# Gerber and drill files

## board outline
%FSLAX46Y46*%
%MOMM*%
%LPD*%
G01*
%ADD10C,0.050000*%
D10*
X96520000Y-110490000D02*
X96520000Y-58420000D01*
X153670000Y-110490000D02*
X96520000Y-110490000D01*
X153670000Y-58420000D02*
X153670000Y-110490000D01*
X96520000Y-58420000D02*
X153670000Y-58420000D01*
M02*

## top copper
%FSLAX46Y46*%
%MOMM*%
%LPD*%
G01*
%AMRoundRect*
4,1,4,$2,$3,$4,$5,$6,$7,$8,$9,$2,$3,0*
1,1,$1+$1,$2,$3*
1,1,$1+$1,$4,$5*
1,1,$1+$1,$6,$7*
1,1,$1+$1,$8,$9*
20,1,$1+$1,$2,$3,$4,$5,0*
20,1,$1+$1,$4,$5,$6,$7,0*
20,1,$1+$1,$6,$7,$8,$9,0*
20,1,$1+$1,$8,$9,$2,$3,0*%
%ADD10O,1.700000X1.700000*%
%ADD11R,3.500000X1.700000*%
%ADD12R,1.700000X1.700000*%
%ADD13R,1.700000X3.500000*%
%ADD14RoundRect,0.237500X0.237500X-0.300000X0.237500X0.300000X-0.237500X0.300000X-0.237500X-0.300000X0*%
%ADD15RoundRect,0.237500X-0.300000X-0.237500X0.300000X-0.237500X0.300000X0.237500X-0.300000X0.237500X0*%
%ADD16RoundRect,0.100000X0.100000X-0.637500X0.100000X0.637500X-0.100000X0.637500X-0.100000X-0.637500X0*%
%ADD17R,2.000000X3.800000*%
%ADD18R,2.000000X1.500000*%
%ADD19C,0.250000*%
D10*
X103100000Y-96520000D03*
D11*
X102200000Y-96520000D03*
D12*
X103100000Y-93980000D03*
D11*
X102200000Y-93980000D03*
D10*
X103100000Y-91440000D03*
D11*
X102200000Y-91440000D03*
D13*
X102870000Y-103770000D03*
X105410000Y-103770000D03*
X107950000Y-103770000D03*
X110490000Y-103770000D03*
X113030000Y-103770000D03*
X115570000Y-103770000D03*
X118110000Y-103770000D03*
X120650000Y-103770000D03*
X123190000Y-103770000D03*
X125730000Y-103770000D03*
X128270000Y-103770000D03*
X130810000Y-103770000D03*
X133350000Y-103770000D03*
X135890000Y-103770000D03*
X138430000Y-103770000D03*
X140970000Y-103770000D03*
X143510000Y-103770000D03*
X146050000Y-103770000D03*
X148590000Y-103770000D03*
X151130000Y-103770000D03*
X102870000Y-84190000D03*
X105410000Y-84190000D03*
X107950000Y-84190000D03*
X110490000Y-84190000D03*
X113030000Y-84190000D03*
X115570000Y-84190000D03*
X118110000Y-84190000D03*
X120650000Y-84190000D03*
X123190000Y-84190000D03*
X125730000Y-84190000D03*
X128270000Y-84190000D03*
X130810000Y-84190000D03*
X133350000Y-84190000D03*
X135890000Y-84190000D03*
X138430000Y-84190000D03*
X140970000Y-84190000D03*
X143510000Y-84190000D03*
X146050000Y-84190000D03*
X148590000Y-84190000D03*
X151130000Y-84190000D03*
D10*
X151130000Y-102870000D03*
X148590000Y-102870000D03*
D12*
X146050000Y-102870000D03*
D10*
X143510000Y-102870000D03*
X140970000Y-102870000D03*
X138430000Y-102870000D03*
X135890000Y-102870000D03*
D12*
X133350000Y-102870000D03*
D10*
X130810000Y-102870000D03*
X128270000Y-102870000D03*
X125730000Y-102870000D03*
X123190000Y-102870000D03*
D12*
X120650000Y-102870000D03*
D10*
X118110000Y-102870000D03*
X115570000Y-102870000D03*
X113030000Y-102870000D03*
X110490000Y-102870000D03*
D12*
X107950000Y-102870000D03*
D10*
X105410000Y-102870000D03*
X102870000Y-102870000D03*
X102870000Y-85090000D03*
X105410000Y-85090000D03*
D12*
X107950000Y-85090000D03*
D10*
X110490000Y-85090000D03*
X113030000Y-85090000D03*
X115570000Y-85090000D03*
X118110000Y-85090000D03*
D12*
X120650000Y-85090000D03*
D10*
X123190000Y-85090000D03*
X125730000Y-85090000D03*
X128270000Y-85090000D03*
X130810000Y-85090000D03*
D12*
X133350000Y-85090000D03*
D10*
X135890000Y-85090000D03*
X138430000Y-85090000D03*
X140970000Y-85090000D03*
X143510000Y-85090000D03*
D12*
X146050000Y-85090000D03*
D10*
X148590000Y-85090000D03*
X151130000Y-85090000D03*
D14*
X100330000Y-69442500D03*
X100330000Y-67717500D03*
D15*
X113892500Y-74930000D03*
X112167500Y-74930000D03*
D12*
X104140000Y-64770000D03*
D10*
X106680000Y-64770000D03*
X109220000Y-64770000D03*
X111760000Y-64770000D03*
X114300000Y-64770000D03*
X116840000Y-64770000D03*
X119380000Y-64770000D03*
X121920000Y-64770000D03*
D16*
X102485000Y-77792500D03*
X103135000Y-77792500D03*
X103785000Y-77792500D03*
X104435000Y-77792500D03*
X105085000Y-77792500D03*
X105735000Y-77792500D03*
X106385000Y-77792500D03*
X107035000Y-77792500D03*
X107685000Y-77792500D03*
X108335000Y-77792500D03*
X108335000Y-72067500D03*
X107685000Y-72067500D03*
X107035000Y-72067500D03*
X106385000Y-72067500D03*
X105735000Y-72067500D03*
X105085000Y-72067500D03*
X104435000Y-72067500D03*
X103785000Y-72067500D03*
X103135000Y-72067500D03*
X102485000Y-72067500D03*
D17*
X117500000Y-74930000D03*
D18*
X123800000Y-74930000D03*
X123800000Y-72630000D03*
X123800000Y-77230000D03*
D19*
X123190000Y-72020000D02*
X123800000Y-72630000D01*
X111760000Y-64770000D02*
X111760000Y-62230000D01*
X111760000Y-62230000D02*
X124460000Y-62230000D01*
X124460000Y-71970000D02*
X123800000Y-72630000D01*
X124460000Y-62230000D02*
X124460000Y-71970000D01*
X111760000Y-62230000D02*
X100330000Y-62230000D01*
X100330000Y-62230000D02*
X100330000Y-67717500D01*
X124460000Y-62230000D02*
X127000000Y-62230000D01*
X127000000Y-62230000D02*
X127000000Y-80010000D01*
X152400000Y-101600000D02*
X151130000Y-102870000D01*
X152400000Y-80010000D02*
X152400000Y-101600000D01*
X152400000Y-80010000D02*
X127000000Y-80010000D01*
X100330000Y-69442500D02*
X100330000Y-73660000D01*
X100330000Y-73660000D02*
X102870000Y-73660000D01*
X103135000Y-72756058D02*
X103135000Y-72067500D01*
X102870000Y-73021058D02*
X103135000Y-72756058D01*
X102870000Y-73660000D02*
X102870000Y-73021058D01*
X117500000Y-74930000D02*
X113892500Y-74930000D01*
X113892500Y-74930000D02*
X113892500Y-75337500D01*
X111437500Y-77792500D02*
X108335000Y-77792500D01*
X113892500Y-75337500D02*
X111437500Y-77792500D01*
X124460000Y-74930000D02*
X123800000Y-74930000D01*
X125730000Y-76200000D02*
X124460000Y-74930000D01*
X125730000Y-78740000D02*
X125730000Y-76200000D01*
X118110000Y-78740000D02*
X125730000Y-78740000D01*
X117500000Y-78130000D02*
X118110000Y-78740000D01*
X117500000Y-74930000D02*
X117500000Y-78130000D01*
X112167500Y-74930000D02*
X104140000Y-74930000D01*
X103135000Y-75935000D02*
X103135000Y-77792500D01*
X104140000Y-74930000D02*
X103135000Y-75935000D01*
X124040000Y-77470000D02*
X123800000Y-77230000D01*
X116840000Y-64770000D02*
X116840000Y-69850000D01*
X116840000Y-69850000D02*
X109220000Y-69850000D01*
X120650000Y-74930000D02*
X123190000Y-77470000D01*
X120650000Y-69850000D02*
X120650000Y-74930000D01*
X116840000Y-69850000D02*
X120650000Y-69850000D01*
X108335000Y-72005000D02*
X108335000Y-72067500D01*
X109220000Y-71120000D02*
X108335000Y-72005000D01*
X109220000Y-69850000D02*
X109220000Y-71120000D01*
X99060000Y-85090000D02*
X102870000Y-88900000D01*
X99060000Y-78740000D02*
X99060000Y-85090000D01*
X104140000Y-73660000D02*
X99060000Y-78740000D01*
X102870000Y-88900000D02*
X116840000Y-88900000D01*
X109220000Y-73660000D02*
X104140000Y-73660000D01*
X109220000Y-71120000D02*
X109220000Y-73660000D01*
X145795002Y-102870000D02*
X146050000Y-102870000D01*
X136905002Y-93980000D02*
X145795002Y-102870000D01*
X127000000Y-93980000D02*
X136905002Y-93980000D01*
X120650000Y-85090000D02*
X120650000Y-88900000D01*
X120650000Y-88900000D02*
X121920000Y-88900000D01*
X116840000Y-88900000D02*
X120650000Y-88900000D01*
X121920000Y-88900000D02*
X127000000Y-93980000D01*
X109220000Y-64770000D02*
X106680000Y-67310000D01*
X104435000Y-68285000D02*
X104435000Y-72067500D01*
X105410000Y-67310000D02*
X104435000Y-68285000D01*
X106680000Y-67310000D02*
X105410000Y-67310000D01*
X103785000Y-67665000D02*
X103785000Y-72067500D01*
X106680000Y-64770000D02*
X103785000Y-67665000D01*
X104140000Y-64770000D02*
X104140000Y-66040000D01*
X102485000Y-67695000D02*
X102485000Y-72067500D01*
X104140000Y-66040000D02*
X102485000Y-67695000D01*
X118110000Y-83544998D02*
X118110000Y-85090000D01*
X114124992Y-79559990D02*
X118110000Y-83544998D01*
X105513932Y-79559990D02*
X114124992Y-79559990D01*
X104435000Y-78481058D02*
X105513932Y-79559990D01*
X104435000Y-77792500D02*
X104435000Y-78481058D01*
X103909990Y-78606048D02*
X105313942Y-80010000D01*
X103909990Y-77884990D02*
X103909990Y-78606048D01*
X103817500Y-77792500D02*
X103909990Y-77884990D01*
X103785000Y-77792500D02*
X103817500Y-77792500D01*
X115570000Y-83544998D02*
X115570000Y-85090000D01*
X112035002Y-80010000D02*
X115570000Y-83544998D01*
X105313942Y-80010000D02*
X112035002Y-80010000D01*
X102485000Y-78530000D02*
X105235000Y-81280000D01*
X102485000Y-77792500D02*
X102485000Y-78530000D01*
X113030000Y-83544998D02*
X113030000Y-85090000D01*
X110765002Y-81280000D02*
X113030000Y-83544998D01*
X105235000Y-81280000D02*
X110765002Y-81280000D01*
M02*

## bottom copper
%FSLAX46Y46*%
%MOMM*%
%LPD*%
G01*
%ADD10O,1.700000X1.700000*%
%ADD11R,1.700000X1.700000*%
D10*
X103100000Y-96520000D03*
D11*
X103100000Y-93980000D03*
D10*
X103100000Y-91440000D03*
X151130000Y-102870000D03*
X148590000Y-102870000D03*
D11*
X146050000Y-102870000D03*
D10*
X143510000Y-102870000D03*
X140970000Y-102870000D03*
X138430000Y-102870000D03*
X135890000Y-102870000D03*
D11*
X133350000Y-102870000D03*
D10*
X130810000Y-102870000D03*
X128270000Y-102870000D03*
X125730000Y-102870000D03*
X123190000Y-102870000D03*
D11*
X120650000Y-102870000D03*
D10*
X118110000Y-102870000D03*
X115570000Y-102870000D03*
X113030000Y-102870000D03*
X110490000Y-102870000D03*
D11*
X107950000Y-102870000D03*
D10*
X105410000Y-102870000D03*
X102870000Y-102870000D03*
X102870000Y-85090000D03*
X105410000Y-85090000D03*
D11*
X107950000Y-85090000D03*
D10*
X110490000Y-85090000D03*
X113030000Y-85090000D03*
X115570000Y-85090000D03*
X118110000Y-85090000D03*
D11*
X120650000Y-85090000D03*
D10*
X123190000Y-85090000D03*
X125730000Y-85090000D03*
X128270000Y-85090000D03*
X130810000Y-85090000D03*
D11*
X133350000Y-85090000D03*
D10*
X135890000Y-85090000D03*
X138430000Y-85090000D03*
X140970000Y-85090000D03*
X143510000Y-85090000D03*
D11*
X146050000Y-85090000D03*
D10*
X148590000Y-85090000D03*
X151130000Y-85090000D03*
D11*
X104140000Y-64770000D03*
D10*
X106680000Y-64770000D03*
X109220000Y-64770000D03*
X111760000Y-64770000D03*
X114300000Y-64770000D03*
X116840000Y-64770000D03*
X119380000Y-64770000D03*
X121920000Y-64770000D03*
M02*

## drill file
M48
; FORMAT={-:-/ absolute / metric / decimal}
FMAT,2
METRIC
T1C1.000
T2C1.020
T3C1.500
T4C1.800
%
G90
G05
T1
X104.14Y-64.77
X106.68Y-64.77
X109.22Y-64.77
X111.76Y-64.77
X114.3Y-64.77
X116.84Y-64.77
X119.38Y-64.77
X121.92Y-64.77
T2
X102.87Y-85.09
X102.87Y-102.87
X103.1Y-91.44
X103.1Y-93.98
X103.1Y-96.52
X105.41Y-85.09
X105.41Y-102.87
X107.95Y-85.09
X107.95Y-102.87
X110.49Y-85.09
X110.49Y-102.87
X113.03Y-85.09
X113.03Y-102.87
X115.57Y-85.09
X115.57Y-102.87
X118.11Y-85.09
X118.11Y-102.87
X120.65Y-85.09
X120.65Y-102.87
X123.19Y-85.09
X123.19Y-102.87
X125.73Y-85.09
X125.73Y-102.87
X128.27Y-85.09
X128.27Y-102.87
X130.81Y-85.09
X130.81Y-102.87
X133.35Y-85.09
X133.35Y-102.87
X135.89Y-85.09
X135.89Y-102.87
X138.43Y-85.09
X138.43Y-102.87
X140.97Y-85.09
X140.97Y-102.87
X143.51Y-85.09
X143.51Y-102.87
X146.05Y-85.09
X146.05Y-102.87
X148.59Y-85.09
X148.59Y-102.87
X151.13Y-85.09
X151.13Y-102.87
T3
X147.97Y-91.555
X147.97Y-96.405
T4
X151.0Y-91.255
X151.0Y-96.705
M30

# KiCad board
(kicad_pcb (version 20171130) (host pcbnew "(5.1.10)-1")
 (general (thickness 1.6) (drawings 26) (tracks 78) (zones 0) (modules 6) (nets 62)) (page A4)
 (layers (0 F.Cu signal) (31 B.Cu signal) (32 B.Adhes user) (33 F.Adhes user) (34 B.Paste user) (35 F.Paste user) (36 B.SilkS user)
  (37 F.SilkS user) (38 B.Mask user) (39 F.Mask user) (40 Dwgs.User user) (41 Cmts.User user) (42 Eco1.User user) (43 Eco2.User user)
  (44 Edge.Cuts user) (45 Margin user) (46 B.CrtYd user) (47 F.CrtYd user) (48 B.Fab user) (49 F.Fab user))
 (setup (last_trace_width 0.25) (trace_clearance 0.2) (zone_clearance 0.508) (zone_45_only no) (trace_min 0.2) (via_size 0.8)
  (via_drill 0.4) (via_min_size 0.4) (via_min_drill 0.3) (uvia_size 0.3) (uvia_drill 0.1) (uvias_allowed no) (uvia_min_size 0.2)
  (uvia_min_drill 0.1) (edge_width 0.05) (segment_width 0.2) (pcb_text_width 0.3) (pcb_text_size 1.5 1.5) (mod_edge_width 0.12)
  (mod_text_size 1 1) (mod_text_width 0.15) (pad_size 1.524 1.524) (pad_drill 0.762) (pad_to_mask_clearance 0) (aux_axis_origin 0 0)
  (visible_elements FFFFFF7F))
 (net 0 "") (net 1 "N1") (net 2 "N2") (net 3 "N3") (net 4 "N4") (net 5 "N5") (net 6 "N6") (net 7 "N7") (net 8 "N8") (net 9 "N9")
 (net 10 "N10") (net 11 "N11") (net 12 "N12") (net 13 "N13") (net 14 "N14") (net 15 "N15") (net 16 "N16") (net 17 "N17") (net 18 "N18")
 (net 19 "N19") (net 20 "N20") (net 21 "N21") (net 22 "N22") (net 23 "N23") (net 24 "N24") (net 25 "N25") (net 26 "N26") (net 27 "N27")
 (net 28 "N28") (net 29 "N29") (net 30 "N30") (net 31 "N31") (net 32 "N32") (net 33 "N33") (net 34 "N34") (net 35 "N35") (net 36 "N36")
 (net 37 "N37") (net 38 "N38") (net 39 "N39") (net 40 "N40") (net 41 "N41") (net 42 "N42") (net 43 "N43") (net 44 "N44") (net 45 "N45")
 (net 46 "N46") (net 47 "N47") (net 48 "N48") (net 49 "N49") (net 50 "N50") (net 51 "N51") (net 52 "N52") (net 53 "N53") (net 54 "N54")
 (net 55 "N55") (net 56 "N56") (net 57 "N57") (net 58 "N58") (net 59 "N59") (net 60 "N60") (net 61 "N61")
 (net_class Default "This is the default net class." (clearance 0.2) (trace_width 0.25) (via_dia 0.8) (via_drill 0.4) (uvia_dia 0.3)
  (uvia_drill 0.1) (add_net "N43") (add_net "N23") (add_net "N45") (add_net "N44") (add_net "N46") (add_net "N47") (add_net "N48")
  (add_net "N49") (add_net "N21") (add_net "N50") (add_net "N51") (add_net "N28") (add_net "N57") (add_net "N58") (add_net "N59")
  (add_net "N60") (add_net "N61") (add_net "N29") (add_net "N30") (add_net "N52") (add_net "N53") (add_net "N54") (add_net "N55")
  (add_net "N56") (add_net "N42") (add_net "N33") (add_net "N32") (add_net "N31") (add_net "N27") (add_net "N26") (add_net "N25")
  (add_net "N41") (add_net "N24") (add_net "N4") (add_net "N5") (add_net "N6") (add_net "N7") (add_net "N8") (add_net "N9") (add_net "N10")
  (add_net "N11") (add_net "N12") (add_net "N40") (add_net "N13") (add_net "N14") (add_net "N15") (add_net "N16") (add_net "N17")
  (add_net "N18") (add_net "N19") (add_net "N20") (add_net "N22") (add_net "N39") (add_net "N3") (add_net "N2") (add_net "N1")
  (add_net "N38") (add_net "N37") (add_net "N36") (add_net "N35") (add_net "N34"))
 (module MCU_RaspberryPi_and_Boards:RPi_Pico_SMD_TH (layer F.Cu) (at 127 93.98 270)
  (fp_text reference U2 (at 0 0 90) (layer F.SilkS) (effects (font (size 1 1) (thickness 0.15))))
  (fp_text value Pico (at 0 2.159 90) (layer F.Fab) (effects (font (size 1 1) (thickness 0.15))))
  (pad 43 thru_hole oval (at 2.54 23.9 270) (size 1.7 1.7) (drill 1.02) (layers *.Cu *.Mask) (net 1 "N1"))
  (pad 43 smd rect (at 2.54 23.9) (size 3.5 1.7) (drill (offset -0.9 0)) (layers F.Cu F.Mask) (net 1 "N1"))
  (pad 42 thru_hole rect (at 0 23.9 270) (size 1.7 1.7) (drill 1.02) (layers *.Cu *.Mask) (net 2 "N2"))
  (pad 42 smd rect (at 0 23.9) (size 3.5 1.7) (drill (offset -0.9 0)) (layers F.Cu F.Mask) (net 2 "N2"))
  (pad 41 thru_hole oval (at -2.54 23.9 270) (size 1.7 1.7) (drill 1.02) (layers *.Cu *.Mask) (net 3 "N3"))
  (pad 41 smd rect (at -2.54 23.9) (size 3.5 1.7) (drill (offset -0.9 0)) (layers F.Cu F.Mask) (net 3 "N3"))
  (pad "" np_thru_hole oval (at 2.425 -20.97 270) (size 1.5 1.5) (drill 1.5) (layers *.Cu *.Mask))
  (pad "" np_thru_hole oval (at -2.425 -20.97 270) (size 1.5 1.5) (drill 1.5) (layers *.Cu *.Mask))
  (pad "" np_thru_hole oval (at 2.725 -24 270) (size 1.8 1.8) (drill 1.8) (layers *.Cu *.Mask))
  (pad "" np_thru_hole oval (at -2.725 -24 270) (size 1.8 1.8) (drill 1.8) (layers *.Cu *.Mask))
  (pad 21 smd rect (at 8.89 24.13 270) (size 3.5 1.7) (drill (offset 0.9 0)) (layers F.Cu F.Mask) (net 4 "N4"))
  (pad 22 smd rect (at 8.89 21.59 270) (size 3.5 1.7) (drill (offset 0.9 0)) (layers F.Cu F.Mask) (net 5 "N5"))
  (pad 23 smd rect (at 8.89 19.05 270) (size 3.5 1.7) (drill (offset 0.9 0)) (layers F.Cu F.Mask) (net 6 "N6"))
  (pad 24 smd rect (at 8.89 16.51 270) (size 3.5 1.7) (drill (offset 0.9 0)) (layers F.Cu F.Mask) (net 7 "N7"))
  (pad 25 smd rect (at 8.89 13.97 270) (size 3.5 1.7) (drill (offset 0.9 0)) (layers F.Cu F.Mask) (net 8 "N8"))
  (pad 26 smd rect (at 8.89 11.43 270) (size 3.5 1.7) (drill (offset 0.9 0)) (layers F.Cu F.Mask) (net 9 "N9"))
  (pad 27 smd rect (at 8.89 8.89 270) (size 3.5 1.7) (drill (offset 0.9 0)) (layers F.Cu F.Mask) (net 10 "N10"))
  (pad 28 smd rect (at 8.89 6.35 270) (size 3.5 1.7) (drill (offset 0.9 0)) (layers F.Cu F.Mask) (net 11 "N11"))
  (pad 29 smd rect (at 8.89 3.81 270) (size 3.5 1.7) (drill (offset 0.9 0)) (layers F.Cu F.Mask) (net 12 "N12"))
  (pad 30 smd rect (at 8.89 1.27 270) (size 3.5 1.7) (drill (offset 0.9 0)) (layers F.Cu F.Mask) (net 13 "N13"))
  (pad 31 smd rect (at 8.89 -1.27 270) (size 3.5 1.7) (drill (offset 0.9 0)) (layers F.Cu F.Mask) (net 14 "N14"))
  (pad 32 smd rect (at 8.89 -3.81 270) (size 3.5 1.7) (drill (offset 0.9 0)) (layers F.Cu F.Mask) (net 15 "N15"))
  (pad 33 smd rect (at 8.89 -6.35 270) (size 3.5 1.7) (drill (offset 0.9 0)) (layers F.Cu F.Mask) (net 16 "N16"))
  (pad 34 smd rect (at 8.89 -8.89 270) (size 3.5 1.7) (drill (offset 0.9 0)) (layers F.Cu F.Mask) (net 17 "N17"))
  (pad 35 smd rect (at 8.89 -11.43 270) (size 3.5 1.7) (drill (offset 0.9 0)) (layers F.Cu F.Mask) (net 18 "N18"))
  (pad 36 smd rect (at 8.89 -13.97 270) (size 3.5 1.7) (drill (offset 0.9 0)) (layers F.Cu F.Mask) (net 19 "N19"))
  (pad 37 smd rect (at 8.89 -16.51 270) (size 3.5 1.7) (drill (offset 0.9 0)) (layers F.Cu F.Mask) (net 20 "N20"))
  (pad 38 smd rect (at 8.89 -19.05 270) (size 3.5 1.7) (drill (offset 0.9 0)) (layers F.Cu F.Mask) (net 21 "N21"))
  (pad 39 smd rect (at 8.89 -21.59 270) (size 3.5 1.7) (drill (offset 0.9 0)) (layers F.Cu F.Mask) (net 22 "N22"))
  (pad 40 smd rect (at 8.89 -24.13 270) (size 3.5 1.7) (drill (offset 0.9 0)) (layers F.Cu F.Mask) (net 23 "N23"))
  (pad 20 smd rect (at -8.89 24.13 270) (size 3.5 1.7) (drill (offset -0.9 0)) (layers F.Cu F.Mask) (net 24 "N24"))
  (pad 19 smd rect (at -8.89 21.59 270) (size 3.5 1.7) (drill (offset -0.9 0)) (layers F.Cu F.Mask) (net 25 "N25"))
  (pad 18 smd rect (at -8.89 19.05 270) (size 3.5 1.7) (drill (offset -0.9 0)) (layers F.Cu F.Mask) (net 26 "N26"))
  (pad 17 smd rect (at -8.89 16.51 270) (size 3.5 1.7) (drill (offset -0.9 0)) (layers F.Cu F.Mask) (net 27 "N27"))
  (pad 16 smd rect (at -8.89 13.97 270) (size 3.5 1.7) (drill (offset -0.9 0)) (layers F.Cu F.Mask) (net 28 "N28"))
  (pad 15 smd rect (at -8.89 11.43 270) (size 3.5 1.7) (drill (offset -0.9 0)) (layers F.Cu F.Mask) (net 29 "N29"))
  (pad 14 smd rect (at -8.89 8.89 270) (size 3.5 1.7) (drill (offset -0.9 0)) (layers F.Cu F.Mask) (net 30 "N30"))
  (pad 13 smd rect (at -8.89 6.35 270) (size 3.5 1.7) (drill (offset -0.9 0)) (layers F.Cu F.Mask) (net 21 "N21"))
  (pad 12 smd rect (at -8.89 3.81 270) (size 3.5 1.7) (drill (offset -0.9 0)) (layers F.Cu F.Mask) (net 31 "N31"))
  (pad 11 smd rect (at -8.89 1.27 270) (size 3.5 1.7) (drill (offset -0.9 0)) (layers F.Cu F.Mask) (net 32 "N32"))
  (pad 10 smd rect (at -8.89 -1.27 270) (size 3.5 1.7) (drill (offset -0.9 0)) (layers F.Cu F.Mask) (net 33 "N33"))
  (pad 9 smd rect (at -8.89 -3.81 270) (size 3.5 1.7) (drill (offset -0.9 0)) (layers F.Cu F.Mask) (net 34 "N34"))
  (pad 8 smd rect (at -8.89 -6.35 270) (size 3.5 1.7) (drill (offset -0.9 0)) (layers F.Cu F.Mask) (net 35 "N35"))
  (pad 7 smd rect (at -8.89 -8.89 270) (size 3.5 1.7) (drill (offset -0.9 0)) (layers F.Cu F.Mask) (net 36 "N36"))
  (pad 6 smd rect (at -8.89 -11.43 270) (size 3.5 1.7) (drill (offset -0.9 0)) (layers F.Cu F.Mask) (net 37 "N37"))
  (pad 5 smd rect (at -8.89 -13.97 270) (size 3.5 1.7) (drill (offset -0.9 0)) (layers F.Cu F.Mask) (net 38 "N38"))
  (pad 4 smd rect (at -8.89 -16.51 270) (size 3.5 1.7) (drill (offset -0.9 0)) (layers F.Cu F.Mask) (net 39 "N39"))
  (pad 3 smd rect (at -8.89 -19.05 270) (size 3.5 1.7) (drill (offset -0.9 0)) (layers F.Cu F.Mask) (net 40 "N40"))
  (pad 2 smd rect (at -8.89 -21.59 270) (size 3.5 1.7) (drill (offset -0.9 0)) (layers F.Cu F.Mask) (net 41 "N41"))
  (pad 1 smd rect (at -8.89 -24.13 270) (size 3.5 1.7) (drill (offset -0.9 0)) (layers F.Cu F.Mask) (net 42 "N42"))
  (pad 40 thru_hole oval (at 8.89 -24.13 270) (size 1.7 1.7) (drill 1.02) (layers *.Cu *.Mask) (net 23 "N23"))
  (pad 39 thru_hole oval (at 8.89 -21.59 270) (size 1.7 1.7) (drill 1.02) (layers *.Cu *.Mask) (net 22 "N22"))
  (pad 38 thru_hole rect (at 8.89 -19.05 270) (size 1.7 1.7) (drill 1.02) (layers *.Cu *.Mask) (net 21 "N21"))
  (pad 37 thru_hole oval (at 8.89 -16.51 270) (size 1.7 1.7) (drill 1.02) (layers *.Cu *.Mask) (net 20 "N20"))
  (pad 36 thru_hole oval (at 8.89 -13.97 270) (size 1.7 1.7) (drill 1.02) (layers *.Cu *.Mask) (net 19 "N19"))
  (pad 35 thru_hole oval (at 8.89 -11.43 270) (size 1.7 1.7) (drill 1.02) (layers *.Cu *.Mask) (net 18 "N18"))
  (pad 34 thru_hole oval (at 8.89 -8.89 270) (size 1.7 1.7) (drill 1.02) (layers *.Cu *.Mask) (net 17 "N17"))
  (pad 33 thru_hole rect (at 8.89 -6.35 270) (size 1.7 1.7) (drill 1.02) (layers *.Cu *.Mask) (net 16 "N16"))
  (pad 32 thru_hole oval (at 8.89 -3.81 270) (size 1.7 1.7) (drill 1.02) (layers *.Cu *.Mask) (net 15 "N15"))
  (pad 31 thru_hole oval (at 8.89 -1.27 270) (size 1.7 1.7) (drill 1.02) (layers *.Cu *.Mask) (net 14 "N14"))
  (pad 30 thru_hole oval (at 8.89 1.27 270) (size 1.7 1.7) (drill 1.02) (layers *.Cu *.Mask) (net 13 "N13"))
  (pad 29 thru_hole oval (at 8.89 3.81 270) (size 1.7 1.7) (drill 1.02) (layers *.Cu *.Mask) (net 12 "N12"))
  (pad 28 thru_hole rect (at 8.89 6.35 270) (size 1.7 1.7) (drill 1.02) (layers *.Cu *.Mask) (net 11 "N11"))
  (pad 27 thru_hole oval (at 8.89 8.89 270) (size 1.7 1.7) (drill 1.02) (layers *.Cu *.Mask) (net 10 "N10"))
  (pad 26 thru_hole oval (at 8.89 11.43 270) (size 1.7 1.7) (drill 1.02) (layers *.Cu *.Mask) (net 9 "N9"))
  (pad 25 thru_hole oval (at 8.89 13.97 270) (size 1.7 1.7) (drill 1.02) (layers *.Cu *.Mask) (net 8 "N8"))
  (pad 24 thru_hole oval (at 8.89 16.51 270) (size 1.7 1.7) (drill 1.02) (layers *.Cu *.Mask) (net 7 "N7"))
  (pad 23 thru_hole rect (at 8.89 19.05 270) (size 1.7 1.7) (drill 1.02) (layers *.Cu *.Mask) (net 6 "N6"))
  (pad 22 thru_hole oval (at 8.89 21.59 270) (size 1.7 1.7) (drill 1.02) (layers *.Cu *.Mask) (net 5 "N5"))
  (pad 21 thru_hole oval (at 8.89 24.13 270) (size 1.7 1.7) (drill 1.02) (layers *.Cu *.Mask) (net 4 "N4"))
  (pad 20 thru_hole oval (at -8.89 24.13 270) (size 1.7 1.7) (drill 1.02) (layers *.Cu *.Mask) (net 24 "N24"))
  (pad 19 thru_hole oval (at -8.89 21.59 270) (size 1.7 1.7) (drill 1.02) (layers *.Cu *.Mask) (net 25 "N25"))
  (pad 18 thru_hole rect (at -8.89 19.05 270) (size 1.7 1.7) (drill 1.02) (layers *.Cu *.Mask) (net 26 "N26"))
  (pad 17 thru_hole oval (at -8.89 16.51 270) (size 1.7 1.7) (drill 1.02) (layers *.Cu *.Mask) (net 27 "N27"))
  (pad 16 thru_hole oval (at -8.89 13.97 270) (size 1.7 1.7) (drill 1.02) (layers *.Cu *.Mask) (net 28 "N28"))
  (pad 15 thru_hole oval (at -8.89 11.43 270) (size 1.7 1.7) (drill 1.02) (layers *.Cu *.Mask) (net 29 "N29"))
  (pad 14 thru_hole oval (at -8.89 8.89 270) (size 1.7 1.7) (drill 1.02) (layers *.Cu *.Mask) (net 30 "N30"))
  (pad 13 thru_hole rect (at -8.89 6.35 270) (size 1.7 1.7) (drill 1.02) (layers *.Cu *.Mask) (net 21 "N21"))
  (pad 12 thru_hole oval (at -8.89 3.81 270) (size 1.7 1.7) (drill 1.02) (layers *.Cu *.Mask) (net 31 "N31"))
  (pad 11 thru_hole oval (at -8.89 1.27 270) (size 1.7 1.7) (drill 1.02) (layers *.Cu *.Mask) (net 32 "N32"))
  (pad 10 thru_hole oval (at -8.89 -1.27 270) (size 1.7 1.7) (drill 1.02) (layers *.Cu *.Mask) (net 33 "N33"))
  (pad 9 thru_hole oval (at -8.89 -3.81 270) (size 1.7 1.7) (drill 1.02) (layers *.Cu *.Mask) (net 34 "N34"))
  (pad 8 thru_hole rect (at -8.89 -6.35 270) (size 1.7 1.7) (drill 1.02) (layers *.Cu *.Mask) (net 35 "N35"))
  (pad 7 thru_hole oval (at -8.89 -8.89 270) (size 1.7 1.7) (drill 1.02) (layers *.Cu *.Mask) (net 36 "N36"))
  (pad 6 thru_hole oval (at -8.89 -11.43 270) (size 1.7 1.7) (drill 1.02) (layers *.Cu *.Mask) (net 37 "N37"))
  (pad 5 thru_hole oval (at -8.89 -13.97 270) (size 1.7 1.7) (drill 1.02) (layers *.Cu *.Mask) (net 38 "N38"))
  (pad 4 thru_hole oval (at -8.89 -16.51 270) (size 1.7 1.7) (drill 1.02) (layers *.Cu *.Mask) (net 39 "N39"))
  (pad 3 thru_hole rect (at -8.89 -19.05 270) (size 1.7 1.7) (drill 1.02) (layers *.Cu *.Mask) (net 40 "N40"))
  (pad 2 thru_hole oval (at -8.89 -21.59 270) (size 1.7 1.7) (drill 1.02) (layers *.Cu *.Mask) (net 41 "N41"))
  (pad 1 thru_hole oval (at -8.89 -24.13 270) (size 1.7 1.7) (drill 1.02) (layers *.Cu *.Mask) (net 42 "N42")))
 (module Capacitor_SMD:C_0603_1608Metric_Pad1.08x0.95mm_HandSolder (layer F.Cu) (at 100.33 68.58 90)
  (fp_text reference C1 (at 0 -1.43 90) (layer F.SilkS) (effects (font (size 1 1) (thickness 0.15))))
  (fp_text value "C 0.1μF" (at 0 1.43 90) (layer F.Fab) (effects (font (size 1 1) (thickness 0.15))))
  (pad 1 smd roundrect (at -0.8625 0 90) (size 1.075 0.95) (layers F.Cu F.Paste F.Mask) (roundrect_rratio 0.25) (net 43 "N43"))
  (pad 2 smd roundrect (at 0.8625 0 90) (size 1.075 0.95) (layers F.Cu F.Paste F.Mask) (roundrect_rratio 0.25) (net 23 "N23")))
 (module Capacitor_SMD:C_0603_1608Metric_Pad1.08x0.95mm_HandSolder (layer F.Cu) (at 113.03 74.93)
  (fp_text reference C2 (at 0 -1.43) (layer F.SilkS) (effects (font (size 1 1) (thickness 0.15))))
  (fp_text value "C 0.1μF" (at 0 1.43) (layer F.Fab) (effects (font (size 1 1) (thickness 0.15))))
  (pad 2 smd roundrect (at 0.8625 0) (size 1.075 0.95) (layers F.Cu F.Paste F.Mask) (roundrect_rratio 0.25) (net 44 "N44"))
  (pad 1 smd roundrect (at -0.8625 0) (size 1.075 0.95) (layers F.Cu F.Paste F.Mask) (roundrect_rratio 0.25) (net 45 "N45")))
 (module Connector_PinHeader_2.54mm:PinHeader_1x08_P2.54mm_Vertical (layer F.Cu) (at 104.14 64.77 90)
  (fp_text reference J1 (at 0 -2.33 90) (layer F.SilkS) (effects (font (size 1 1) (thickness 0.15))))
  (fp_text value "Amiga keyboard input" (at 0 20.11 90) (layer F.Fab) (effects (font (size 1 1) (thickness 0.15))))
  (pad 1 thru_hole rect (at 0 0 90) (size 1.7 1.7) (drill 1) (layers *.Cu *.Mask) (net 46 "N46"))
  (pad 2 thru_hole oval (at 0 2.54 90) (size 1.7 1.7) (drill 1) (layers *.Cu *.Mask) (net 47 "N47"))
  (pad 3 thru_hole oval (at 0 5.08 90) (size 1.7 1.7) (drill 1) (layers *.Cu *.Mask) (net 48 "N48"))
  (pad 4 thru_hole oval (at 0 7.62 90) (size 1.7 1.7) (drill 1) (layers *.Cu *.Mask) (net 23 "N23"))
  (pad 5 thru_hole oval (at 0 10.16 90) (size 1.7 1.7) (drill 1) (layers *.Cu *.Mask) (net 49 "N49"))
  (pad 6 thru_hole oval (at 0 12.7 90) (size 1.7 1.7) (drill 1) (layers *.Cu *.Mask) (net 21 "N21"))
  (pad 7 thru_hole oval (at 0 15.24 90) (size 1.7 1.7) (drill 1) (layers *.Cu *.Mask) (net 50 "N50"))
  (pad 8 thru_hole oval (at 0 17.78 90) (size 1.7 1.7) (drill 1) (layers *.Cu *.Mask) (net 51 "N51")))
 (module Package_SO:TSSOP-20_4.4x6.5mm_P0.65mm (layer F.Cu) (at 105.41 74.93 90)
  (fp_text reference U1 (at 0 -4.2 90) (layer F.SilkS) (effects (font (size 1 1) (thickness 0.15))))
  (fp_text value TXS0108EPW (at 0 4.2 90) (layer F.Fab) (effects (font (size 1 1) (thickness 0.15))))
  (pad 1 smd roundrect (at -2.8625 -2.925 90) (size 1.475 0.4) (layers F.Cu F.Paste F.Mask) (roundrect_rratio 0.25) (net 28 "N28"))
  (pad 2 smd roundrect (at -2.8625 -2.275 90) (size 1.475 0.4) (layers F.Cu F.Paste F.Mask) (roundrect_rratio 0.25) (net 45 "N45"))
  (pad 3 smd roundrect (at -2.8625 -1.625 90) (size 1.475 0.4) (layers F.Cu F.Paste F.Mask) (roundrect_rratio 0.25) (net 29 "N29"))
  (pad 4 smd roundrect (at -2.8625 -0.975 90) (size 1.475 0.4) (layers F.Cu F.Paste F.Mask) (roundrect_rratio 0.25) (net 30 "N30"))
  (pad 5 smd roundrect (at -2.8625 -0.325 90) (size 1.475 0.4) (layers F.Cu F.Paste F.Mask) (roundrect_rratio 0.25) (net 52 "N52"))
  (pad 6 smd roundrect (at -2.8625 0.325 90) (size 1.475 0.4) (layers F.Cu F.Paste F.Mask) (roundrect_rratio 0.25) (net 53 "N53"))
  (pad 7 smd roundrect (at -2.8625 0.975 90) (size 1.475 0.4) (layers F.Cu F.Paste F.Mask) (roundrect_rratio 0.25) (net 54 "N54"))
  (pad 8 smd roundrect (at -2.8625 1.625 90) (size 1.475 0.4) (layers F.Cu F.Paste F.Mask) (roundrect_rratio 0.25) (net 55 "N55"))
  (pad 9 smd roundrect (at -2.8625 2.275 90) (size 1.475 0.4) (layers F.Cu F.Paste F.Mask) (roundrect_rratio 0.25) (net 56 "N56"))
  (pad 10 smd roundrect (at -2.8625 2.925 90) (size 1.475 0.4) (layers F.Cu F.Paste F.Mask) (roundrect_rratio 0.25) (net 44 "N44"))
  (pad 11 smd roundrect (at 2.8625 2.925 90) (size 1.475 0.4) (layers F.Cu F.Paste F.Mask) (roundrect_rratio 0.25) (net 21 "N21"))
  (pad 12 smd roundrect (at 2.8625 2.275 90) (size 1.475 0.4) (layers F.Cu F.Paste F.Mask) (roundrect_rratio 0.25) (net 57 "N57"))
  (pad 13 smd roundrect (at 2.8625 1.625 90) (size 1.475 0.4) (layers F.Cu F.Paste F.Mask) (roundrect_rratio 0.25) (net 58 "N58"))
  (pad 14 smd roundrect (at 2.8625 0.975 90) (size 1.475 0.4) (layers F.Cu F.Paste F.Mask) (roundrect_rratio 0.25) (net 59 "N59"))
  (pad 15 smd roundrect (at 2.8625 0.325 90) (size 1.475 0.4) (layers F.Cu F.Paste F.Mask) (roundrect_rratio 0.25) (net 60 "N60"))
  (pad 16 smd roundrect (at 2.8625 -0.325 90) (size 1.475 0.4) (layers F.Cu F.Paste F.Mask) (roundrect_rratio 0.25) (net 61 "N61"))
  (pad 17 smd roundrect (at 2.8625 -0.975 90) (size 1.475 0.4) (layers F.Cu F.Paste F.Mask) (roundrect_rratio 0.25) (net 48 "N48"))
  (pad 18 smd roundrect (at 2.8625 -1.625 90) (size 1.475 0.4) (layers F.Cu F.Paste F.Mask) (roundrect_rratio 0.25) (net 47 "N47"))
  (pad 19 smd roundrect (at 2.8625 -2.275 90) (size 1.475 0.4) (layers F.Cu F.Paste F.Mask) (roundrect_rratio 0.25) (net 43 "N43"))
  (pad 20 smd roundrect (at 2.8625 -2.925 90) (size 1.475 0.4) (layers F.Cu F.Paste F.Mask) (roundrect_rratio 0.25) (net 46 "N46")))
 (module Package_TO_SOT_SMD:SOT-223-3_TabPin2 (layer F.Cu) (at 120.65 74.93 180)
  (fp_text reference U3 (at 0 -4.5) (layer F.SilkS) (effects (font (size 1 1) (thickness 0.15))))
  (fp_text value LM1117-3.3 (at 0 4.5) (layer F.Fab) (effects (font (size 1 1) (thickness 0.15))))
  (pad 2 smd rect (at 3.15 0 180) (size 2 3.8) (layers F.Cu F.Paste F.Mask) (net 44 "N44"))
  (pad 2 smd rect (at -3.15 0 180) (size 2 1.5) (layers F.Cu F.Paste F.Mask) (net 44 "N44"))
  (pad 3 smd rect (at -3.15 2.3 180) (size 2 1.5) (layers F.Cu F.Paste F.Mask) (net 23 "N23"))
  (pad 1 smd rect (at -3.15 -2.3 180) (size 2 1.5) (layers F.Cu F.Paste F.Mask) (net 21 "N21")))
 (gr_line (start 96.52 110.49) (end 96.52 58.42) (layer Edge.Cuts) (width 0.05))
 (gr_line (start 153.67 110.49) (end 96.52 110.49) (layer Edge.Cuts) (width 0.05))
 (gr_line (start 153.67 58.42) (end 153.67 110.49) (layer Edge.Cuts) (width 0.05))
 (gr_line (start 96.52 58.42) (end 153.67 58.42) (layer Edge.Cuts) (width 0.05))
 (segment (start 123.19 72.02) (end 123.8 72.63) (width 0.25) (layer F.Cu) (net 23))
 (segment (start 111.76 64.77) (end 111.76 62.23) (width 0.25) (layer F.Cu) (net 23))
 (segment (start 111.76 62.23) (end 124.46 62.23) (width 0.25) (layer F.Cu) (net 23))
 (segment (start 124.46 71.97) (end 123.8 72.63) (width 0.25) (layer F.Cu) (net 23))
 (segment (start 124.46 62.23) (end 124.46 71.97) (width 0.25) (layer F.Cu) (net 23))
 (segment (start 111.76 62.23) (end 100.33 62.23) (width 0.25) (layer F.Cu) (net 23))
 (segment (start 100.33 62.23) (end 100.33 67.7175) (width 0.25) (layer F.Cu) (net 23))
 (segment (start 124.46 62.23) (end 127 62.23) (width 0.25) (layer F.Cu) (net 23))
 (segment (start 127 62.23) (end 127 80.01) (width 0.25) (layer F.Cu) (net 23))
 (segment (start 152.4 101.6) (end 151.13 102.87) (width 0.25) (layer F.Cu) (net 23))
 (segment (start 152.4 80.01) (end 152.4 101.6) (width 0.25) (layer F.Cu) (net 23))
 (segment (start 152.4 80.01) (end 127 80.01) (width 0.25) (layer F.Cu) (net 23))
 (segment (start 100.33 69.4425) (end 100.33 73.66) (width 0.25) (layer F.Cu) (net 43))
 (segment (start 100.33 73.66) (end 102.87 73.66) (width 0.25) (layer F.Cu) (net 43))
 (segment (start 103.135 72.756058) (end 103.135 72.0675) (width 0.25) (layer F.Cu) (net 43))
 (segment (start 102.87 73.021058) (end 103.135 72.756058) (width 0.25) (layer F.Cu) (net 43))
 (segment (start 102.87 73.66) (end 102.87 73.021058) (width 0.25) (layer F.Cu) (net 43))
 (segment (start 117.5 74.93) (end 113.8925 74.93) (width 0.25) (layer F.Cu) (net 44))
 (segment (start 113.8925 74.93) (end 113.8925 75.3375) (width 0.25) (layer F.Cu) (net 44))
 (segment (start 111.4375 77.7925) (end 108.335 77.7925) (width 0.25) (layer F.Cu) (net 44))
 (segment (start 113.8925 75.3375) (end 111.4375 77.7925) (width 0.25) (layer F.Cu) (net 44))
 (segment (start 124.46 74.93) (end 123.8 74.93) (width 0.25) (layer F.Cu) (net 44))
 (segment (start 125.73 76.2) (end 124.46 74.93) (width 0.25) (layer F.Cu) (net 44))
 (segment (start 125.73 78.74) (end 125.73 76.2) (width 0.25) (layer F.Cu) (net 44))
 (segment (start 118.11 78.74) (end 125.73 78.74) (width 0.25) (layer F.Cu) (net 44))
 (segment (start 117.5 78.13) (end 118.11 78.74) (width 0.25) (layer F.Cu) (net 44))
 (segment (start 117.5 74.93) (end 117.5 78.13) (width 0.25) (layer F.Cu) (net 44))
 (segment (start 112.1675 74.93) (end 104.14 74.93) (width 0.25) (layer F.Cu) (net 45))
 (segment (start 103.135 75.935) (end 103.135 77.7925) (width 0.25) (layer F.Cu) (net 45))
 (segment (start 104.14 74.93) (end 103.135 75.935) (width 0.25) (layer F.Cu) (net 45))
 (segment (start 124.04 77.47) (end 123.8 77.23) (width 0.25) (layer F.Cu) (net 21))
 (segment (start 116.84 64.77) (end 116.84 69.85) (width 0.25) (layer F.Cu) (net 21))
 (segment (start 116.84 69.85) (end 109.22 69.85) (width 0.25) (layer F.Cu) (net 21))
 (segment (start 120.65 74.93) (end 123.19 77.47) (width 0.25) (layer F.Cu) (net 21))
 (segment (start 120.65 69.85) (end 120.65 74.93) (width 0.25) (layer F.Cu) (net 21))
 (segment (start 116.84 69.85) (end 120.65 69.85) (width 0.25) (layer F.Cu) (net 21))
 (segment (start 108.335 72.005) (end 108.335 72.0675) (width 0.25) (layer F.Cu) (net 21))
 (segment (start 109.22 71.12) (end 108.335 72.005) (width 0.25) (layer F.Cu) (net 21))
 (segment (start 109.22 69.85) (end 109.22 71.12) (width 0.25) (layer F.Cu) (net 21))
 (segment (start 99.06 85.09) (end 102.87 88.9) (width 0.25) (layer F.Cu) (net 21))
 (segment (start 99.06 78.74) (end 99.06 85.09) (width 0.25) (layer F.Cu) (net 21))
 (segment (start 104.14 73.66) (end 99.06 78.74) (width 0.25) (layer F.Cu) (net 21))
 (segment (start 102.87 88.9) (end 116.84 88.9) (width 0.25) (layer F.Cu) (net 21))
 (segment (start 109.22 73.66) (end 104.14 73.66) (width 0.25) (layer F.Cu) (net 21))
 (segment (start 109.22 71.12) (end 109.22 73.66) (width 0.25) (layer F.Cu) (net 21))
 (segment (start 145.795002 102.87) (end 146.05 102.87) (width 0.25) (layer F.Cu) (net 21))
 (segment (start 136.905002 93.98) (end 145.795002 102.87) (width 0.25) (layer F.Cu) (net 21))
 (segment (start 127 93.98) (end 136.905002 93.98) (width 0.25) (layer F.Cu) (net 21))
 (segment (start 120.65 85.09) (end 120.65 88.9) (width 0.25) (layer F.Cu) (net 21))
 (segment (start 120.65 88.9) (end 121.92 88.9) (width 0.25) (layer F.Cu) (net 21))
 (segment (start 116.84 88.9) (end 120.65 88.9) (width 0.25) (layer F.Cu) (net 21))
 (segment (start 121.92 88.9) (end 127 93.98) (width 0.25) (layer F.Cu) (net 21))
 (segment (start 109.22 64.77) (end 106.68 67.31) (width 0.25) (layer F.Cu) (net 48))
 (segment (start 104.435 68.285) (end 104.435 72.0675) (width 0.25) (layer F.Cu) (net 48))
 (segment (start 105.41 67.31) (end 104.435 68.285) (width 0.25) (layer F.Cu) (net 48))
 (segment (start 106.68 67.31) (end 105.41 67.31) (width 0.25) (layer F.Cu) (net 48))
 (segment (start 103.785 67.665) (end 103.785 72.0675) (width 0.25) (layer F.Cu) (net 47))
 (segment (start 106.68 64.77) (end 103.785 67.665) (width 0.25) (layer F.Cu) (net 47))
 (segment (start 104.14 64.77) (end 104.14 66.04) (width 0.25) (layer F.Cu) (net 46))
 (segment (start 102.485 67.695) (end 102.485 72.0675) (width 0.25) (layer F.Cu) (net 46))
 (segment (start 104.14 66.04) (end 102.485 67.695) (width 0.25) (layer F.Cu) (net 46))
 (segment (start 118.11 83.544998) (end 118.11 85.09) (width 0.25) (layer F.Cu) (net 30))
 (segment (start 114.124992 79.55999) (end 118.11 83.544998) (width 0.25) (layer F.Cu) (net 30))
 (segment (start 105.513932 79.55999) (end 114.124992 79.55999) (width 0.25) (layer F.Cu) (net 30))
 (segment (start 104.435 78.481058) (end 105.513932 79.55999) (width 0.25) (layer F.Cu) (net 30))
 (segment (start 104.435 77.7925) (end 104.435 78.481058) (width 0.25) (layer F.Cu) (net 30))
 (segment (start 103.90999 78.606048) (end 105.313942 80.01) (width 0.25) (layer F.Cu) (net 29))
 (segment (start 103.90999 77.88499) (end 103.90999 78.606048) (width 0.25) (layer F.Cu) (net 29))
 (segment (start 103.8175 77.7925) (end 103.90999 77.88499) (width 0.25) (layer F.Cu) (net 29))
 (segment (start 103.785 77.7925) (end 103.8175 77.7925) (width 0.25) (layer F.Cu) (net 29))
 (segment (start 115.57 83.544998) (end 115.57 85.09) (width 0.25) (layer F.Cu) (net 29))
 (segment (start 112.035002 80.01) (end 115.57 83.544998) (width 0.25) (layer F.Cu) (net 29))
 (segment (start 105.313942 80.01) (end 112.035002 80.01) (width 0.25) (layer F.Cu) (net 29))
 (segment (start 102.485 78.53) (end 105.235 81.28) (width 0.25) (layer F.Cu) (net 28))
 (segment (start 102.485 77.7925) (end 102.485 78.53) (width 0.25) (layer F.Cu) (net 28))
 (segment (start 113.03 83.544998) (end 113.03 85.09) (width 0.25) (layer F.Cu) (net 28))
 (segment (start 110.765002 81.28) (end 113.03 83.544998) (width 0.25) (layer F.Cu) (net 28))
 (segment (start 105.235 81.28) (end 110.765002 81.28) (width 0.25) (layer F.Cu) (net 28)))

